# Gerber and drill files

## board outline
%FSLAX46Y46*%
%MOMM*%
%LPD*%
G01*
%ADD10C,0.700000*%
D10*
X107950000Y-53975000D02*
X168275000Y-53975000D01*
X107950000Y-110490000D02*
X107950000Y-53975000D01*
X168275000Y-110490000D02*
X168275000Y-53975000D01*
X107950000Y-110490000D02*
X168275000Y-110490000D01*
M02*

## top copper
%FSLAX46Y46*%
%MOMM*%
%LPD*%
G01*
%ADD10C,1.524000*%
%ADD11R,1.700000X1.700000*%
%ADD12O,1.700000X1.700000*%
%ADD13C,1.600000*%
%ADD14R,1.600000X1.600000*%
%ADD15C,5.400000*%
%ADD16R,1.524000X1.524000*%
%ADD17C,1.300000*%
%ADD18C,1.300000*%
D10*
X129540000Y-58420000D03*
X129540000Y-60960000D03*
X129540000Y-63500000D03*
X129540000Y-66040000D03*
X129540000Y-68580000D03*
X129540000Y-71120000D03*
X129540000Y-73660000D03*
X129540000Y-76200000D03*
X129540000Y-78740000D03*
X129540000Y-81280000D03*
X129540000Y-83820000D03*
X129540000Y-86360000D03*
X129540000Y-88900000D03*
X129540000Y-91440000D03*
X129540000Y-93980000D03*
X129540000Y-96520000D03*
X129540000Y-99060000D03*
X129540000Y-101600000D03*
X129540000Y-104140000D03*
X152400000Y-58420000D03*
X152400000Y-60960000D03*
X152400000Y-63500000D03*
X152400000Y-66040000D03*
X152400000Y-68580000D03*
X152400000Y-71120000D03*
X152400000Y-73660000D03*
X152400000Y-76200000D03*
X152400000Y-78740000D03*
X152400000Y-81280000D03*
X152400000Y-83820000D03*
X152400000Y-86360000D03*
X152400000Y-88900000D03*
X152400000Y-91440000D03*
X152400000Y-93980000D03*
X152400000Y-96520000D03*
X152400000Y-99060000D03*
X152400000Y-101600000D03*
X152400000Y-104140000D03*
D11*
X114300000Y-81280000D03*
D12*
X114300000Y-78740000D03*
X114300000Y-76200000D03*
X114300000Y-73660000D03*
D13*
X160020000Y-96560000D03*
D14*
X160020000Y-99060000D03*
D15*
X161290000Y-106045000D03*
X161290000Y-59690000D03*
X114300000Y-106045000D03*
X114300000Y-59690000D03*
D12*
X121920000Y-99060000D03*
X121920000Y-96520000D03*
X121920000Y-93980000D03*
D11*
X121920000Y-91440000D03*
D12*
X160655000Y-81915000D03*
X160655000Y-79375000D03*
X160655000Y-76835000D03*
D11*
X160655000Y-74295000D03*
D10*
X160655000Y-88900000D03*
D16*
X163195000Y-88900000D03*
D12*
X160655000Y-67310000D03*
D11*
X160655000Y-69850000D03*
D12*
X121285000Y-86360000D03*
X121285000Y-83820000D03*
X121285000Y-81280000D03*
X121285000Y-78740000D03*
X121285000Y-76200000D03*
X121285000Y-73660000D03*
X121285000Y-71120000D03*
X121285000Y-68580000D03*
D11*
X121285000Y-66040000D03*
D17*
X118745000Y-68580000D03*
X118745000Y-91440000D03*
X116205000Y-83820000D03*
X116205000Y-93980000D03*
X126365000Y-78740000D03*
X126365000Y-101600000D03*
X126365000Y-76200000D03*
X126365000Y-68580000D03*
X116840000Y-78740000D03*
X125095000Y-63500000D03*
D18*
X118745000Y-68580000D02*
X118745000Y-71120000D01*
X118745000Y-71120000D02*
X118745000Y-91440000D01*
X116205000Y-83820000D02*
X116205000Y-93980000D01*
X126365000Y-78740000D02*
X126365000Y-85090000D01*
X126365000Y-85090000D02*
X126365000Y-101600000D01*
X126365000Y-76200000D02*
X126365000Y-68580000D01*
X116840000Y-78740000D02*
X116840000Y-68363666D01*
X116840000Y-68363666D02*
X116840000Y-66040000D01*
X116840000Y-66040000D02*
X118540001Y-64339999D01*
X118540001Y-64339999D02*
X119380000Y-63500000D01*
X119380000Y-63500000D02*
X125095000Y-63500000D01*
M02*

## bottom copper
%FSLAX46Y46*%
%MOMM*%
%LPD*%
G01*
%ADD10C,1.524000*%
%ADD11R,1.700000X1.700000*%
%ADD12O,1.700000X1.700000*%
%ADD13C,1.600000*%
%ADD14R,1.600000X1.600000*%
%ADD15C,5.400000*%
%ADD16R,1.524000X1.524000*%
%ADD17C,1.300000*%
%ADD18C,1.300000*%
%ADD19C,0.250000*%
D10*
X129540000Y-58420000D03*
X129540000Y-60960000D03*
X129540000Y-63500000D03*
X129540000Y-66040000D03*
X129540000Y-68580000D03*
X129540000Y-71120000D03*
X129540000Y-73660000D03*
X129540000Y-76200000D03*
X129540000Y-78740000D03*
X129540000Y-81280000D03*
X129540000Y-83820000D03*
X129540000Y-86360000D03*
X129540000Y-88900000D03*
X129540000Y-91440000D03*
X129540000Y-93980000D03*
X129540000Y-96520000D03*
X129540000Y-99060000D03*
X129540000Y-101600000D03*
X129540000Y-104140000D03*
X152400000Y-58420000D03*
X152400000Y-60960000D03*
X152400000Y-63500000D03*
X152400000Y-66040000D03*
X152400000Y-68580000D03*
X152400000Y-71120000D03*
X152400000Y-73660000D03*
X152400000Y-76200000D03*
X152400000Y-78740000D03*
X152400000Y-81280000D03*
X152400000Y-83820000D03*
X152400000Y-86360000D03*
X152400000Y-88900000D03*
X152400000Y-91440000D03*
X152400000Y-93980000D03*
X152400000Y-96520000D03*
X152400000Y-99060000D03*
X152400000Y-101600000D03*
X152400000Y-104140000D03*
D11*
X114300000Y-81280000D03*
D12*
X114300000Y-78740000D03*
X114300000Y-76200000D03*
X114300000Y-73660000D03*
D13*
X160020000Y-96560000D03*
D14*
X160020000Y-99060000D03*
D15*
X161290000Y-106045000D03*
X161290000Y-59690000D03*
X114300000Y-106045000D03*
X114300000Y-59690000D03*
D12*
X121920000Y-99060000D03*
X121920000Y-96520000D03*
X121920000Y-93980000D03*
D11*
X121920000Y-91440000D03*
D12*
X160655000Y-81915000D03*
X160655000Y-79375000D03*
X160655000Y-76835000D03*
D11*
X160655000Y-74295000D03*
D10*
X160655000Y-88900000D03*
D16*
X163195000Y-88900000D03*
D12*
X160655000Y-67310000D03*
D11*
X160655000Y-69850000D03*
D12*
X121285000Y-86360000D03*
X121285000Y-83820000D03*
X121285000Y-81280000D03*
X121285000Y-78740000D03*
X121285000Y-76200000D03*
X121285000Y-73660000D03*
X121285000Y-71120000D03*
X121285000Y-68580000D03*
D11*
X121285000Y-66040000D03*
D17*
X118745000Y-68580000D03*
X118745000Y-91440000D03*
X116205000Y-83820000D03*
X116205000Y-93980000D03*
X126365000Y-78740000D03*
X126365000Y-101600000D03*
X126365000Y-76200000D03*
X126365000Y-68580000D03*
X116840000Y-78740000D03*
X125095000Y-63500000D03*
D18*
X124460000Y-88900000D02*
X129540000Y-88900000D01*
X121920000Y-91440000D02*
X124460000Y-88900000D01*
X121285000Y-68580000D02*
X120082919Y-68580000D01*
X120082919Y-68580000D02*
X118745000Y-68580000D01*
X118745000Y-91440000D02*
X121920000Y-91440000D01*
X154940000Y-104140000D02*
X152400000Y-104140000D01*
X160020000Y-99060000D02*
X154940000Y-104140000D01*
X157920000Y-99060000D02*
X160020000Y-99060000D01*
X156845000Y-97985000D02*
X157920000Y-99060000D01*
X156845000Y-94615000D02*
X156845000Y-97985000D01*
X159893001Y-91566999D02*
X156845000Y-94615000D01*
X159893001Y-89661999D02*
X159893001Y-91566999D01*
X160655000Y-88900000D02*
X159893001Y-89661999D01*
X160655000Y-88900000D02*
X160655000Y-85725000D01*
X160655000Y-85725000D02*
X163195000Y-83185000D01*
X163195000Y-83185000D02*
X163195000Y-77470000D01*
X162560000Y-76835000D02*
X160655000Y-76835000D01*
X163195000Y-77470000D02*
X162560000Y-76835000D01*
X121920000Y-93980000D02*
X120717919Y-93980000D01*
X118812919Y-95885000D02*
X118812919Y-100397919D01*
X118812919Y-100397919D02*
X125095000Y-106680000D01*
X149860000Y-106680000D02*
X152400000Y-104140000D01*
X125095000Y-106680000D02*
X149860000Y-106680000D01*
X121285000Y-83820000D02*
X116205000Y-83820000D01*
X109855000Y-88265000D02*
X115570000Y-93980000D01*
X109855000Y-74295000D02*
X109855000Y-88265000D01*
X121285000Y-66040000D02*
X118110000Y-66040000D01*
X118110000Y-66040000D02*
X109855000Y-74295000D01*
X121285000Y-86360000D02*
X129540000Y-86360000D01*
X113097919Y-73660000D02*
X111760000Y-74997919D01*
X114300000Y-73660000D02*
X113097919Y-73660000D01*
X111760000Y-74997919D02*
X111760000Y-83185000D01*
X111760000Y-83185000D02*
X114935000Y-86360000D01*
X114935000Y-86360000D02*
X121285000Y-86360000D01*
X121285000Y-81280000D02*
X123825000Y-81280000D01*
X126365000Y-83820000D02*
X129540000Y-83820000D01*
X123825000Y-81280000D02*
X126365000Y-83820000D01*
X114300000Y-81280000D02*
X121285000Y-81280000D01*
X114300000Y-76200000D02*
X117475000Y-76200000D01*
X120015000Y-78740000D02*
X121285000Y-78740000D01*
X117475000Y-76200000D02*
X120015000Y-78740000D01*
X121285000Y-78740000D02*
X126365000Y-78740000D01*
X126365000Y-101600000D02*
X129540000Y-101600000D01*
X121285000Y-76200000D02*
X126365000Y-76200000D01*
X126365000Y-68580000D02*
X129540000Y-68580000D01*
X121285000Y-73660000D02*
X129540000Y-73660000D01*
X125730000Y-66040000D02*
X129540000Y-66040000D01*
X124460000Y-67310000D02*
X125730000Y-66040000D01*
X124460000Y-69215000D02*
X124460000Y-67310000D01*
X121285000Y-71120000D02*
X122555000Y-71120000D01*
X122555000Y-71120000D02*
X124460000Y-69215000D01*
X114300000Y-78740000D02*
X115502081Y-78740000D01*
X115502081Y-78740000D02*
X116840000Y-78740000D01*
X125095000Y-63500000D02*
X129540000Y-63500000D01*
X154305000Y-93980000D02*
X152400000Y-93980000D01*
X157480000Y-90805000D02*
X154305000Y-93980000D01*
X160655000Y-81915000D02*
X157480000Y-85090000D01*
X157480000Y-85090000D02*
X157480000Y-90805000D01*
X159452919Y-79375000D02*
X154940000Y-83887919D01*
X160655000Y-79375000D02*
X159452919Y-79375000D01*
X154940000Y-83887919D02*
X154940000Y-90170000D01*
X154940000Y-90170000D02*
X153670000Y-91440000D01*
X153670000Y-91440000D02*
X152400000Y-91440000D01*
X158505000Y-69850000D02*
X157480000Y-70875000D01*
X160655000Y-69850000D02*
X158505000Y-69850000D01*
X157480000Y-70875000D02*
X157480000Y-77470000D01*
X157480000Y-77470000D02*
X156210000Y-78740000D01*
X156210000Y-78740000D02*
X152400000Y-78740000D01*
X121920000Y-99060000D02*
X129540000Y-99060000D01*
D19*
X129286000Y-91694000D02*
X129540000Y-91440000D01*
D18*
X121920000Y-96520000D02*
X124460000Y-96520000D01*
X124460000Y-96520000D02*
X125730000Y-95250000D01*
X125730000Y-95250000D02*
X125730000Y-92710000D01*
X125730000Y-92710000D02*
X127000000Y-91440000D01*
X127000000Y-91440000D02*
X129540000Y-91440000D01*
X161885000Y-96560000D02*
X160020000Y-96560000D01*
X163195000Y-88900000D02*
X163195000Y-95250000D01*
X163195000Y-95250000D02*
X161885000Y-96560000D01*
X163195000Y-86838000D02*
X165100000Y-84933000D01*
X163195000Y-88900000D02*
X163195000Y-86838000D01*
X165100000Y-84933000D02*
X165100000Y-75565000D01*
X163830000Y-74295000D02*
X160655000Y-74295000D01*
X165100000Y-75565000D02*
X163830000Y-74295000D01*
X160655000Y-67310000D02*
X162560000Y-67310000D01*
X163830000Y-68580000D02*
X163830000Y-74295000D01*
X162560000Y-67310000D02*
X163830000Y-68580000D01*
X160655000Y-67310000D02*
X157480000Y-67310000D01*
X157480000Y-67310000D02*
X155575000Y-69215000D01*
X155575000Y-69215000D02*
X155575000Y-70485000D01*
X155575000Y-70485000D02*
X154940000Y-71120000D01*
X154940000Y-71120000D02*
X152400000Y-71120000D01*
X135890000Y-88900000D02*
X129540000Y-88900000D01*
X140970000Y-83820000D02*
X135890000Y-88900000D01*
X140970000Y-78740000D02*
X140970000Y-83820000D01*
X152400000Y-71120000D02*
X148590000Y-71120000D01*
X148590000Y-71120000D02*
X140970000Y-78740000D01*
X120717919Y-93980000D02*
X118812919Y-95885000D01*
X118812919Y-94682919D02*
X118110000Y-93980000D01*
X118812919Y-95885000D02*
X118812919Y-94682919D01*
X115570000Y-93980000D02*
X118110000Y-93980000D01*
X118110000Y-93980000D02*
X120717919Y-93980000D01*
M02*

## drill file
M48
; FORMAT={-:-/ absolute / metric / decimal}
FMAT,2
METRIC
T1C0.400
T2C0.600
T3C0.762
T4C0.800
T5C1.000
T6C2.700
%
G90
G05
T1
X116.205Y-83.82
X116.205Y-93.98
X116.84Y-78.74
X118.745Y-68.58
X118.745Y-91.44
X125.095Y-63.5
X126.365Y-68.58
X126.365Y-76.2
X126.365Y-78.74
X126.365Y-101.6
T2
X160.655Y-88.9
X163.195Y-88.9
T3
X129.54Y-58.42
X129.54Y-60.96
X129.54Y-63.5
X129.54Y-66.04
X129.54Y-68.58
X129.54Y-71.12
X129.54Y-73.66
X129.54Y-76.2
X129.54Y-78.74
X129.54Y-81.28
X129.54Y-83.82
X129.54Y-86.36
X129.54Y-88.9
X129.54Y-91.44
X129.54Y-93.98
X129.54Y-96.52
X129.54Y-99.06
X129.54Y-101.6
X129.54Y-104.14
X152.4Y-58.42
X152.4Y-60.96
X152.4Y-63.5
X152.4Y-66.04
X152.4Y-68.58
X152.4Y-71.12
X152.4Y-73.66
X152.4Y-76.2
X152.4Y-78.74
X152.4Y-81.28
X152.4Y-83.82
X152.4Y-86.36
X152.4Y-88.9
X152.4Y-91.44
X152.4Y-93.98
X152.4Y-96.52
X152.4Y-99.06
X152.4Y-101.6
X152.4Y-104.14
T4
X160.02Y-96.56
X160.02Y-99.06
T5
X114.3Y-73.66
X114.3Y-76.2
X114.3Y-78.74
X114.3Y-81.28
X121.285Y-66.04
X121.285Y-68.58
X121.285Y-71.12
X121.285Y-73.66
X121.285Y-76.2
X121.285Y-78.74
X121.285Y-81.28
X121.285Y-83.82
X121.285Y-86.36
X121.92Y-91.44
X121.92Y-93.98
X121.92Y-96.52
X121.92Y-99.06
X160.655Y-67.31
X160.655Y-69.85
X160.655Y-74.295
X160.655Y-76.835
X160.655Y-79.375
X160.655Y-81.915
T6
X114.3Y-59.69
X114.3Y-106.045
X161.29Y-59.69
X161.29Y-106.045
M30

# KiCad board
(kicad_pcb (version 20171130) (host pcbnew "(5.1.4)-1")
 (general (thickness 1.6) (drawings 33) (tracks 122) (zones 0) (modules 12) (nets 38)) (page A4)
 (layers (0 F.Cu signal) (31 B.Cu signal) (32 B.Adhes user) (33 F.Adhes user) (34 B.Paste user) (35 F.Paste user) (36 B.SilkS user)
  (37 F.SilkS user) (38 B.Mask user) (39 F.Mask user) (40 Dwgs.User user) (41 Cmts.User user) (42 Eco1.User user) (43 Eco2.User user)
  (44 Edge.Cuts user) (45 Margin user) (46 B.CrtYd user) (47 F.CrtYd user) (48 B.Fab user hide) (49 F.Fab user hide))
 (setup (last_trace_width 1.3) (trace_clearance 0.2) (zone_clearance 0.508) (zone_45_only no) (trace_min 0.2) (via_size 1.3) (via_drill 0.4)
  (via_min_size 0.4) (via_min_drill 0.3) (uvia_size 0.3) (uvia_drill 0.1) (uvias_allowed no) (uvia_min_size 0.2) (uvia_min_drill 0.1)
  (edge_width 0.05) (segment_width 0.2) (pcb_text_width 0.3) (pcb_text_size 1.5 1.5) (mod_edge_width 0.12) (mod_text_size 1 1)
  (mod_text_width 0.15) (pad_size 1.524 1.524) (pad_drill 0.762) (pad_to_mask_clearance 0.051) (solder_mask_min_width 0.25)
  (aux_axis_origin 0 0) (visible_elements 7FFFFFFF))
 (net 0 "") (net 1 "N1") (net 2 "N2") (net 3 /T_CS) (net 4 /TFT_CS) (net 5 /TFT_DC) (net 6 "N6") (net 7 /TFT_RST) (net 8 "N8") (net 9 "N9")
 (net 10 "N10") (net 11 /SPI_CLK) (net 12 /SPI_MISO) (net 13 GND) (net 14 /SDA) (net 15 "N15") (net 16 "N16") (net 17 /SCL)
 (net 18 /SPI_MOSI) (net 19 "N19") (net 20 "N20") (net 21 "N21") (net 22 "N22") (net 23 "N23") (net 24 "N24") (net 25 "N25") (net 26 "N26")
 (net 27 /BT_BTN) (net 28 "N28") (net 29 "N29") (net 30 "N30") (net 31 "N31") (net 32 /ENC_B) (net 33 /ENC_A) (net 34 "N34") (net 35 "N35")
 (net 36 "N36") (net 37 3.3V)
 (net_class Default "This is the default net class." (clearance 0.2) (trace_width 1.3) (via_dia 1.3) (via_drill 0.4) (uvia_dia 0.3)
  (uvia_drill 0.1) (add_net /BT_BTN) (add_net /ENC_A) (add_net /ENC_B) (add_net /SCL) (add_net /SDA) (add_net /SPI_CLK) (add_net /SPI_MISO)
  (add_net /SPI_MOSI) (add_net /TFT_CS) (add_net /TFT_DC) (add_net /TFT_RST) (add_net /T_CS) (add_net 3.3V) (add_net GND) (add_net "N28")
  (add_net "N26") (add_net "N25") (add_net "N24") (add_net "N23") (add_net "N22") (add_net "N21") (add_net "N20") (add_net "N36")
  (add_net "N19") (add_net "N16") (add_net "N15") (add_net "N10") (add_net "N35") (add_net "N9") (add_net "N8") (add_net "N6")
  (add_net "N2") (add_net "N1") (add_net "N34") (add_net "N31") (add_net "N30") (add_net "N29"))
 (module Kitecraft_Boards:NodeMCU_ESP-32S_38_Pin (layer F.Cu) (at 140.97 81.28 180)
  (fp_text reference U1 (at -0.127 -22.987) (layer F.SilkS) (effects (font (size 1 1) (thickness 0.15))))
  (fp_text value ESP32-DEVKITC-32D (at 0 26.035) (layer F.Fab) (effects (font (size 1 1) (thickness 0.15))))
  (pad 38 thru_hole circle (at 11.43 22.86 180) (size 1.524 1.524) (drill 0.762) (layers *.Cu *.Mask) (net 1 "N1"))
  (pad 37 thru_hole circle (at 11.43 20.32 180) (size 1.524 1.524) (drill 0.762) (layers *.Cu *.Mask) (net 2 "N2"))
  (pad 36 thru_hole circle (at 11.43 17.78 180) (size 1.524 1.524) (drill 0.762) (layers *.Cu *.Mask) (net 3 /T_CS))
  (pad 35 thru_hole circle (at 11.43 15.24 180) (size 1.524 1.524) (drill 0.762) (layers *.Cu *.Mask) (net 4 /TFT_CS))
  (pad 34 thru_hole circle (at 11.43 12.7 180) (size 1.524 1.524) (drill 0.762) (layers *.Cu *.Mask) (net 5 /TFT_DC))
  (pad 33 thru_hole circle (at 11.43 10.16 180) (size 1.524 1.524) (drill 0.762) (layers *.Cu *.Mask) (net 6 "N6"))
  (pad 32 thru_hole circle (at 11.43 7.62 180) (size 1.524 1.524) (drill 0.762) (layers *.Cu *.Mask) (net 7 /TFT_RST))
  (pad 31 thru_hole circle (at 11.43 5.08 180) (size 1.524 1.524) (drill 0.762) (layers *.Cu *.Mask) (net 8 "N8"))
  (pad 30 thru_hole circle (at 11.43 2.54 180) (size 1.524 1.524) (drill 0.762) (layers *.Cu *.Mask) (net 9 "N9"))
  (pad 29 thru_hole circle (at 11.43 0 180) (size 1.524 1.524) (drill 0.762) (layers *.Cu *.Mask) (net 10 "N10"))
  (pad 28 thru_hole circle (at 11.43 -2.54 180) (size 1.524 1.524) (drill 0.762) (layers *.Cu *.Mask) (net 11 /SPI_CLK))
  (pad 27 thru_hole circle (at 11.43 -5.08 180) (size 1.524 1.524) (drill 0.762) (layers *.Cu *.Mask) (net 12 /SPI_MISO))
  (pad 26 thru_hole circle (at 11.43 -7.62 180) (size 1.524 1.524) (drill 0.762) (layers *.Cu *.Mask) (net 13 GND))
  (pad 25 thru_hole circle (at 11.43 -10.16 180) (size 1.524 1.524) (drill 0.762) (layers *.Cu *.Mask) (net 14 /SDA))
  (pad 24 thru_hole circle (at 11.43 -12.7 180) (size 1.524 1.524) (drill 0.762) (layers *.Cu *.Mask) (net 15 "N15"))
  (pad 23 thru_hole circle (at 11.43 -15.24 180) (size 1.524 1.524) (drill 0.762) (layers *.Cu *.Mask) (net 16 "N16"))
  (pad 22 thru_hole circle (at 11.43 -17.78 180) (size 1.524 1.524) (drill 0.762) (layers *.Cu *.Mask) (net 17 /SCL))
  (pad 21 thru_hole circle (at 11.43 -20.32 180) (size 1.524 1.524) (drill 0.762) (layers *.Cu *.Mask) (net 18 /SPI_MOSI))
  (pad 20 thru_hole circle (at 11.43 -22.86 180) (size 1.524 1.524) (drill 0.762) (layers *.Cu *.Mask) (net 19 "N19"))
  (pad 19 thru_hole circle (at -11.43 22.86 180) (size 1.524 1.524) (drill 0.762) (layers *.Cu *.Mask) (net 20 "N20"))
  (pad 18 thru_hole circle (at -11.43 20.32 180) (size 1.524 1.524) (drill 0.762) (layers *.Cu *.Mask) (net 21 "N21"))
  (pad 17 thru_hole circle (at -11.43 17.78 180) (size 1.524 1.524) (drill 0.762) (layers *.Cu *.Mask) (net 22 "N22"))
  (pad 16 thru_hole circle (at -11.43 15.24 180) (size 1.524 1.524) (drill 0.762) (layers *.Cu *.Mask) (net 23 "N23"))
  (pad 15 thru_hole circle (at -11.43 12.7 180) (size 1.524 1.524) (drill 0.762) (layers *.Cu *.Mask) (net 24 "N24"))
  (pad 14 thru_hole circle (at -11.43 10.16 180) (size 1.524 1.524) (drill 0.762) (layers *.Cu *.Mask) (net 13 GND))
  (pad 13 thru_hole circle (at -11.43 7.62 180) (size 1.524 1.524) (drill 0.762) (layers *.Cu *.Mask) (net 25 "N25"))
  (pad 12 thru_hole circle (at -11.43 5.08 180) (size 1.524 1.524) (drill 0.762) (layers *.Cu *.Mask) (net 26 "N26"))
  (pad 11 thru_hole circle (at -11.43 2.54 180) (size 1.524 1.524) (drill 0.762) (layers *.Cu *.Mask) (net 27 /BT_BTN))
  (pad 10 thru_hole circle (at -11.43 0 180) (size 1.524 1.524) (drill 0.762) (layers *.Cu *.Mask) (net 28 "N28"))
  (pad 9 thru_hole circle (at -11.43 -2.54 180) (size 1.524 1.524) (drill 0.762) (layers *.Cu *.Mask) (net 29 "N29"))
  (pad 8 thru_hole circle (at -11.43 -5.08 180) (size 1.524 1.524) (drill 0.762) (layers *.Cu *.Mask) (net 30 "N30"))
  (pad 7 thru_hole circle (at -11.43 -7.62 180) (size 1.524 1.524) (drill 0.762) (layers *.Cu *.Mask) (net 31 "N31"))
  (pad 6 thru_hole circle (at -11.43 -10.16 180) (size 1.524 1.524) (drill 0.762) (layers *.Cu *.Mask) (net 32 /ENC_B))
  (pad 5 thru_hole circle (at -11.43 -12.7 180) (size 1.524 1.524) (drill 0.762) (layers *.Cu *.Mask) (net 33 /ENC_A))
  (pad 4 thru_hole circle (at -11.43 -15.24 180) (size 1.524 1.524) (drill 0.762) (layers *.Cu *.Mask) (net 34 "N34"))
  (pad 3 thru_hole circle (at -11.43 -17.78 180) (size 1.524 1.524) (drill 0.762) (layers *.Cu *.Mask) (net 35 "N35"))
  (pad 2 thru_hole circle (at -11.43 -20.32 180) (size 1.524 1.524) (drill 0.762) (layers *.Cu *.Mask) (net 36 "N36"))
  (pad 1 thru_hole circle (at -11.43 -22.86 180) (size 1.524 1.524) (drill 0.762) (layers *.Cu *.Mask) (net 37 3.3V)))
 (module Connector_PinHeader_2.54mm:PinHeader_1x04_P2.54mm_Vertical (layer F.Cu) (at 114.3 81.28 180)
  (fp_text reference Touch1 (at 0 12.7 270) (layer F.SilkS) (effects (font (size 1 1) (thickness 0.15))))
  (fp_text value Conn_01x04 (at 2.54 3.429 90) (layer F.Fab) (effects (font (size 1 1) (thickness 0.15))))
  (pad 1 thru_hole rect (at 0 0 180) (size 1.7 1.7) (drill 1) (layers *.Cu *.Mask) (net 11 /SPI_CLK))
  (pad 2 thru_hole oval (at 0 2.54 180) (size 1.7 1.7) (drill 1) (layers *.Cu *.Mask) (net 3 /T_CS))
  (pad 3 thru_hole oval (at 0 5.08 180) (size 1.7 1.7) (drill 1) (layers *.Cu *.Mask) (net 18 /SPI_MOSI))
  (pad 4 thru_hole oval (at 0 7.62 180) (size 1.7 1.7) (drill 1) (layers *.Cu *.Mask) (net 12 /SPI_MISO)))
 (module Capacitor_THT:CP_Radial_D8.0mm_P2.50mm (layer F.Cu) (at 160.02 99.06 90)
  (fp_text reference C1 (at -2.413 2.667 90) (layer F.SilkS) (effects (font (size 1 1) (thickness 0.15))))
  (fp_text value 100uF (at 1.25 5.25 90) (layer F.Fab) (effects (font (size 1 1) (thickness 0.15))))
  (pad 2 thru_hole circle (at 2.5 0 90) (size 1.6 1.6) (drill 0.8) (layers *.Cu *.Mask) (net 13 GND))
  (pad 1 thru_hole rect (at 0 0 90) (size 1.6 1.6) (drill 0.8) (layers *.Cu *.Mask) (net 37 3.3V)))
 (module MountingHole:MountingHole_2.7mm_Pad (layer F.Cu) (at 161.29 106.045)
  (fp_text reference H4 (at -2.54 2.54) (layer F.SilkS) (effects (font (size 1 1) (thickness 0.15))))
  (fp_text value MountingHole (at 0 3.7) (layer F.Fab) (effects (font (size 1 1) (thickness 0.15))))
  (pad 1 thru_hole circle (at 0 0) (size 5.4 5.4) (drill 2.7) (layers *.Cu *.Mask)))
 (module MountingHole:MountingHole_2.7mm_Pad (layer F.Cu) (at 161.29 59.69)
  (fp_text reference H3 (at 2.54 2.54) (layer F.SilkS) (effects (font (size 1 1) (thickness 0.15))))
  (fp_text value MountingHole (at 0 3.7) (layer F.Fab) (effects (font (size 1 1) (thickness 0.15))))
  (pad 1 thru_hole circle (at 0 0) (size 5.4 5.4) (drill 2.7) (layers *.Cu *.Mask)))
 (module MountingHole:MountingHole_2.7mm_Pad (layer F.Cu) (at 114.3 106.045)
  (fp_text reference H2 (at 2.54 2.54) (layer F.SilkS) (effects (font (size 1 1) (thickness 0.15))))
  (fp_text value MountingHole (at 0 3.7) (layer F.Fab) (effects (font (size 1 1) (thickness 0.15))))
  (pad 1 thru_hole circle (at 0 0) (size 5.4 5.4) (drill 2.7) (layers *.Cu *.Mask)))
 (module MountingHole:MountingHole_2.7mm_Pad (layer F.Cu) (at 114.3 59.69)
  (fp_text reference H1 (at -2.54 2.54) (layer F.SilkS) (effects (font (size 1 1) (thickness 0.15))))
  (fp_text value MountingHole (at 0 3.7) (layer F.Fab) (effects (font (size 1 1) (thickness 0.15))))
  (pad 1 thru_hole circle (at 0 0) (size 5.4 5.4) (drill 2.7) (layers *.Cu *.Mask)))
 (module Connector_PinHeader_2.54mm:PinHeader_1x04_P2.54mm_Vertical (layer F.Cu) (at 121.92 91.44)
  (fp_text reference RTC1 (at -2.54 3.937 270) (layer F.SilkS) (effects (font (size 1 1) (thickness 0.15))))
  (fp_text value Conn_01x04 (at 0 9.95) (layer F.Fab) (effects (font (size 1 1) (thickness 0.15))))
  (pad 4 thru_hole oval (at 0 7.62) (size 1.7 1.7) (drill 1) (layers *.Cu *.Mask) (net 17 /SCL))
  (pad 3 thru_hole oval (at 0 5.08) (size 1.7 1.7) (drill 1) (layers *.Cu *.Mask) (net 14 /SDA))
  (pad 2 thru_hole oval (at 0 2.54) (size 1.7 1.7) (drill 1) (layers *.Cu *.Mask) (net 37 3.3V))
  (pad 1 thru_hole rect (at 0 0) (size 1.7 1.7) (drill 1) (layers *.Cu *.Mask) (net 13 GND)))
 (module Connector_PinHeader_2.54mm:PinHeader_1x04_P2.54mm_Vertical (layer F.Cu) (at 160.655 74.295)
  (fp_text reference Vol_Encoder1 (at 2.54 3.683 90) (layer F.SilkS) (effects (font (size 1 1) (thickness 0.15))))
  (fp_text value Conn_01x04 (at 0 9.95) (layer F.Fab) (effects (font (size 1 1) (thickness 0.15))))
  (pad 4 thru_hole oval (at 0 7.62) (size 1.7 1.7) (drill 1) (layers *.Cu *.Mask) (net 33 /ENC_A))
  (pad 3 thru_hole oval (at 0 5.08) (size 1.7 1.7) (drill 1) (layers *.Cu *.Mask) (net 32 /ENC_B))
  (pad 2 thru_hole oval (at 0 2.54) (size 1.7 1.7) (drill 1) (layers *.Cu *.Mask) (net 37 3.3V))
  (pad 1 thru_hole rect (at 0 0) (size 1.7 1.7) (drill 1) (layers *.Cu *.Mask) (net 13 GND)))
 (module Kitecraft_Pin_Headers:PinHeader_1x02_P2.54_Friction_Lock (layer F.Cu) (at 160.655 88.9 270)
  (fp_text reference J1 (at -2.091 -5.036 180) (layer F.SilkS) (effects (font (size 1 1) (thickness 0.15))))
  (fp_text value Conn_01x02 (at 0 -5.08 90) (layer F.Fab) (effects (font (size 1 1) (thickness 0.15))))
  (pad 2 thru_hole circle (at 0 0 270) (size 1.524 1.524) (drill 0.6) (layers *.Cu *.Mask) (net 37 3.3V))
  (pad 1 thru_hole rect (at 0 -2.54 270) (size 1.524 1.524) (drill 0.6) (layers *.Cu *.Mask) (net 13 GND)))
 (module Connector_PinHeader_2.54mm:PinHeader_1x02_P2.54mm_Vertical (layer F.Cu) (at 160.655 69.85 180)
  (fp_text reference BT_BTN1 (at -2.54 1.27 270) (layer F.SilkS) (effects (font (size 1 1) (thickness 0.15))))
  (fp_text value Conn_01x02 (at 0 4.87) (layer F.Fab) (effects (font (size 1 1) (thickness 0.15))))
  (pad 2 thru_hole oval (at 0 2.54 180) (size 1.7 1.7) (drill 1) (layers *.Cu *.Mask) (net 13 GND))
  (pad 1 thru_hole rect (at 0 0 180) (size 1.7 1.7) (drill 1) (layers *.Cu *.Mask) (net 27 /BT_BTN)))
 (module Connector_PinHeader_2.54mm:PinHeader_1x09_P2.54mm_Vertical (layer F.Cu) (at 121.285 66.04)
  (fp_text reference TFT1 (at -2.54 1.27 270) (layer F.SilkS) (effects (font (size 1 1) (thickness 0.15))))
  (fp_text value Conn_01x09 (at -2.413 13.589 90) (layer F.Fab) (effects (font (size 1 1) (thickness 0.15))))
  (pad 9 thru_hole oval (at 0 20.32) (size 1.7 1.7) (drill 1) (layers *.Cu *.Mask) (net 12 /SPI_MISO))
  (pad 8 thru_hole oval (at 0 17.78) (size 1.7 1.7) (drill 1) (layers *.Cu *.Mask) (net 37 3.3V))
  (pad 7 thru_hole oval (at 0 15.24) (size 1.7 1.7) (drill 1) (layers *.Cu *.Mask) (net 11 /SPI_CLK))
  (pad 6 thru_hole oval (at 0 12.7) (size 1.7 1.7) (drill 1) (layers *.Cu *.Mask) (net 18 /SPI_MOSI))
  (pad 5 thru_hole oval (at 0 10.16) (size 1.7 1.7) (drill 1) (layers *.Cu *.Mask) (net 5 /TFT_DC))
  (pad 4 thru_hole oval (at 0 7.62) (size 1.7 1.7) (drill 1) (layers *.Cu *.Mask) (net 7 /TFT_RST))
  (pad 3 thru_hole oval (at 0 5.08) (size 1.7 1.7) (drill 1) (layers *.Cu *.Mask) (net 4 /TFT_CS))
  (pad 2 thru_hole oval (at 0 2.54) (size 1.7 1.7) (drill 1) (layers *.Cu *.Mask) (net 13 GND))
  (pad 1 thru_hole rect (at 0 0) (size 1.7 1.7) (drill 1) (layers *.Cu *.Mask) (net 37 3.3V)))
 (gr_line (start 107.95 53.975) (end 168.275 53.975) (layer Edge.Cuts) (width 0.7))
 (gr_line (start 107.95 110.49) (end 107.95 53.975) (layer Edge.Cuts) (width 0.7))
 (gr_line (start 168.275 110.49) (end 168.275 53.975) (layer Edge.Cuts) (width 0.7))
 (gr_line (start 107.95 110.49) (end 168.275 110.49) (layer Edge.Cuts) (width 0.7))
 (segment (start 124.46 88.9) (end 129.54 88.9) (width 1.3) (layer B.Cu) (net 13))
 (segment (start 121.92 91.44) (end 124.46 88.9) (width 1.3) (layer B.Cu) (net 13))
 (segment (start 121.285 68.58) (end 120.082919 68.58) (width 1.3) (layer B.Cu) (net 13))
 (via (at 118.745 68.58) (size 1.3) (drill 0.4) (layers F.Cu B.Cu) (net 13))
 (segment (start 120.082919 68.58) (end 118.745 68.58) (width 1.3) (layer B.Cu) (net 13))
 (segment (start 118.745 68.58) (end 118.745 71.12) (width 1.3) (layer F.Cu) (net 13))
 (segment (start 118.745 71.12) (end 118.745 91.44) (width 1.3) (layer F.Cu) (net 13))
 (via (at 118.745 91.44) (size 1.3) (drill 0.4) (layers F.Cu B.Cu) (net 13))
 (segment (start 118.745 91.44) (end 121.92 91.44) (width 1.3) (layer B.Cu) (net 13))
 (segment (start 154.94 104.14) (end 152.4 104.14) (width 1.3) (layer B.Cu) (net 37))
 (segment (start 160.02 99.06) (end 154.94 104.14) (width 1.3) (layer B.Cu) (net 37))
 (segment (start 157.92 99.06) (end 160.02 99.06) (width 1.3) (layer B.Cu) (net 37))
 (segment (start 156.845 97.985) (end 157.92 99.06) (width 1.3) (layer B.Cu) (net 37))
 (segment (start 156.845 94.615) (end 156.845 97.985) (width 1.3) (layer B.Cu) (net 37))
 (segment (start 159.893001 91.566999) (end 156.845 94.615) (width 1.3) (layer B.Cu) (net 37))
 (segment (start 159.893001 89.661999) (end 159.893001 91.566999) (width 1.3) (layer B.Cu) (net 37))
 (segment (start 160.655 88.9) (end 159.893001 89.661999) (width 1.3) (layer B.Cu) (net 37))
 (segment (start 160.655 88.9) (end 160.655 85.725) (width 1.3) (layer B.Cu) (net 37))
 (segment (start 160.655 85.725) (end 163.195 83.185) (width 1.3) (layer B.Cu) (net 37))
 (segment (start 163.195 83.185) (end 163.195 77.47) (width 1.3) (layer B.Cu) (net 37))
 (segment (start 162.56 76.835) (end 160.655 76.835) (width 1.3) (layer B.Cu) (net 37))
 (segment (start 163.195 77.47) (end 162.56 76.835) (width 1.3) (layer B.Cu) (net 37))
 (segment (start 121.92 93.98) (end 120.717919 93.98) (width 1.3) (layer B.Cu) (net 37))
 (segment (start 118.812919 95.885) (end 118.812919 100.397919) (width 1.3) (layer B.Cu) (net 37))
 (segment (start 118.812919 100.397919) (end 125.095 106.68) (width 1.3) (layer B.Cu) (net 37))
 (segment (start 149.86 106.68) (end 152.4 104.14) (width 1.3) (layer B.Cu) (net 37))
 (segment (start 125.095 106.68) (end 149.86 106.68) (width 1.3) (layer B.Cu) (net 37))
 (segment (start 121.285 83.82) (end 116.205 83.82) (width 1.3) (layer B.Cu) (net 37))
 (via (at 116.205 83.82) (size 1.3) (drill 0.4) (layers F.Cu B.Cu) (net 37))
 (segment (start 116.205 83.82) (end 116.205 93.98) (width 1.3) (layer F.Cu) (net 37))
 (via (at 116.205 93.98) (size 1.3) (drill 0.4) (layers F.Cu B.Cu) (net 37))
 (segment (start 109.855 88.265) (end 115.57 93.98) (width 1.3) (layer B.Cu) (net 37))
 (segment (start 109.855 74.295) (end 109.855 88.265) (width 1.3) (layer B.Cu) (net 37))
 (segment (start 121.285 66.04) (end 118.11 66.04) (width 1.3) (layer B.Cu) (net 37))
 (segment (start 118.11 66.04) (end 109.855 74.295) (width 1.3) (layer B.Cu) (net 37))
 (segment (start 121.285 86.36) (end 129.54 86.36) (width 1.3) (layer B.Cu) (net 12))
 (segment (start 113.097919 73.66) (end 111.76 74.997919) (width 1.3) (layer B.Cu) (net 12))
 (segment (start 114.3 73.66) (end 113.097919 73.66) (width 1.3) (layer B.Cu) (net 12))
 (segment (start 111.76 74.997919) (end 111.76 83.185) (width 1.3) (layer B.Cu) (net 12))
 (segment (start 111.76 83.185) (end 114.935 86.36) (width 1.3) (layer B.Cu) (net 12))
 (segment (start 114.935 86.36) (end 121.285 86.36) (width 1.3) (layer B.Cu) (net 12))
 (segment (start 121.285 81.28) (end 123.825 81.28) (width 1.3) (layer B.Cu) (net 11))
 (segment (start 126.365 83.82) (end 129.54 83.82) (width 1.3) (layer B.Cu) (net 11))
 (segment (start 123.825 81.28) (end 126.365 83.82) (width 1.3) (layer B.Cu) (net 11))
 (segment (start 114.3 81.28) (end 121.285 81.28) (width 1.3) (layer B.Cu) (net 11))
 (segment (start 114.3 76.2) (end 117.475 76.2) (width 1.3) (layer B.Cu) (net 18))
 (segment (start 120.015 78.74) (end 121.285 78.74) (width 1.3) (layer B.Cu) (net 18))
 (segment (start 117.475 76.2) (end 120.015 78.74) (width 1.3) (layer B.Cu) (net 18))
 (segment (start 121.285 78.74) (end 126.365 78.74) (width 1.3) (layer B.Cu) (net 18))
 (via (at 126.365 78.74) (size 1.3) (drill 0.4) (layers F.Cu B.Cu) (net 18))
 (segment (start 126.365 78.74) (end 126.365 85.09) (width 1.3) (layer F.Cu) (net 18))
 (segment (start 126.365 85.09) (end 126.365 101.6) (width 1.3) (layer F.Cu) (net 18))
 (via (at 126.365 101.6) (size 1.3) (drill 0.4) (layers F.Cu B.Cu) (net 18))
 (segment (start 126.365 101.6) (end 129.54 101.6) (width 1.3) (layer B.Cu) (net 18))
 (segment (start 121.285 76.2) (end 126.365 76.2) (width 1.3) (layer B.Cu) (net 5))
 (via (at 126.365 76.2) (size 1.3) (drill 0.4) (layers F.Cu B.Cu) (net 5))
 (segment (start 126.365 76.2) (end 126.365 68.58) (width 1.3) (layer F.Cu) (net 5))
 (via (at 126.365 68.58) (size 1.3) (drill 0.4) (layers F.Cu B.Cu) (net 5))
 (segment (start 126.365 68.58) (end 129.54 68.58) (width 1.3) (layer B.Cu) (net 5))
 (segment (start 121.285 73.66) (end 129.54 73.66) (width 1.3) (layer B.Cu) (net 7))
 (segment (start 125.73 66.04) (end 129.54 66.04) (width 1.3) (layer B.Cu) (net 4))
 (segment (start 124.46 67.31) (end 125.73 66.04) (width 1.3) (layer B.Cu) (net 4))
 (segment (start 124.46 69.215) (end 124.46 67.31) (width 1.3) (layer B.Cu) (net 4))
 (segment (start 121.285 71.12) (end 122.555 71.12) (width 1.3) (layer B.Cu) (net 4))
 (segment (start 122.555 71.12) (end 124.46 69.215) (width 1.3) (layer B.Cu) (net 4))
 (segment (start 114.3 78.74) (end 115.502081 78.74) (width 1.3) (layer B.Cu) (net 3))
 (via (at 116.84 78.74) (size 1.3) (drill 0.4) (layers F.Cu B.Cu) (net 3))
 (segment (start 115.502081 78.74) (end 116.84 78.74) (width 1.3) (layer B.Cu) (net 3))
 (segment (start 116.84 78.74) (end 116.84 68.363666) (width 1.3) (layer F.Cu) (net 3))
 (segment (start 116.84 68.363666) (end 116.84 66.04) (width 1.3) (layer F.Cu) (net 3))
 (segment (start 116.84 66.04) (end 118.540001 64.339999) (width 1.3) (layer F.Cu) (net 3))
 (segment (start 118.540001 64.339999) (end 119.38 63.5) (width 1.3) (layer F.Cu) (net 3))
 (via (at 125.095 63.5) (size 1.3) (drill 0.4) (layers F.Cu B.Cu) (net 3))
 (segment (start 119.38 63.5) (end 125.095 63.5) (width 1.3) (layer F.Cu) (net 3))
 (segment (start 125.095 63.5) (end 129.54 63.5) (width 1.3) (layer B.Cu) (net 3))
 (segment (start 154.305 93.98) (end 152.4 93.98) (width 1.3) (layer B.Cu) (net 33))
 (segment (start 157.48 90.805) (end 154.305 93.98) (width 1.3) (layer B.Cu) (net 33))
 (segment (start 160.655 81.915) (end 157.48 85.09) (width 1.3) (layer B.Cu) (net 33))
 (segment (start 157.48 85.09) (end 157.48 90.805) (width 1.3) (layer B.Cu) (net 33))
 (segment (start 159.452919 79.375) (end 154.94 83.887919) (width 1.3) (layer B.Cu) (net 32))
 (segment (start 160.655 79.375) (end 159.452919 79.375) (width 1.3) (layer B.Cu) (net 32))
 (segment (start 154.94 83.887919) (end 154.94 90.17) (width 1.3) (layer B.Cu) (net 32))
 (segment (start 154.94 90.17) (end 153.67 91.44) (width 1.3) (layer B.Cu) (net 32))
 (segment (start 153.67 91.44) (end 152.4 91.44) (width 1.3) (layer B.Cu) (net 32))
 (segment (start 158.505 69.85) (end 157.48 70.875) (width 1.3) (layer B.Cu) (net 27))
 (segment (start 160.655 69.85) (end 158.505 69.85) (width 1.3) (layer B.Cu) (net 27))
 (segment (start 157.48 70.875) (end 157.48 77.47) (width 1.3) (layer B.Cu) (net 27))
 (segment (start 157.48 77.47) (end 156.21 78.74) (width 1.3) (layer B.Cu) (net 27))
 (segment (start 156.21 78.74) (end 152.4 78.74) (width 1.3) (layer B.Cu) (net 27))
 (segment (start 121.92 99.06) (end 129.54 99.06) (width 1.3) (layer B.Cu) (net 17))
 (segment (start 129.286 91.694) (end 129.54 91.44) (width 0.25) (layer B.Cu) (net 14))
 (segment (start 121.92 96.52) (end 124.46 96.52) (width 1.3) (layer B.Cu) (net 14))
 (segment (start 124.46 96.52) (end 125.73 95.25) (width 1.3) (layer B.Cu) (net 14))
 (segment (start 125.73 95.25) (end 125.73 92.71) (width 1.3) (layer B.Cu) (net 14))
 (segment (start 125.73 92.71) (end 127 91.44) (width 1.3) (layer B.Cu) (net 14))
 (segment (start 127 91.44) (end 129.54 91.44) (width 1.3) (layer B.Cu) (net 14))
 (segment (start 161.885 96.56) (end 160.02 96.56) (width 1.3) (layer B.Cu) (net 13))
 (segment (start 163.195 88.9) (end 163.195 95.25) (width 1.3) (layer B.Cu) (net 13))
 (segment (start 163.195 95.25) (end 161.885 96.56) (width 1.3) (layer B.Cu) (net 13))
 (segment (start 163.195 86.838) (end 165.1 84.933) (width 1.3) (layer B.Cu) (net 13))
 (segment (start 163.195 88.9) (end 163.195 86.838) (width 1.3) (layer B.Cu) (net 13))
 (segment (start 165.1 84.933) (end 165.1 75.565) (width 1.3) (layer B.Cu) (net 13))
 (segment (start 163.83 74.295) (end 160.655 74.295) (width 1.3) (layer B.Cu) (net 13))
 (segment (start 165.1 75.565) (end 163.83 74.295) (width 1.3) (layer B.Cu) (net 13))
 (segment (start 160.655 67.31) (end 162.56 67.31) (width 1.3) (layer B.Cu) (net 13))
 (segment (start 163.83 68.58) (end 163.83 74.295) (width 1.3) (layer B.Cu) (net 13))
 (segment (start 162.56 67.31) (end 163.83 68.58) (width 1.3) (layer B.Cu) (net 13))
 (segment (start 160.655 67.31) (end 157.48 67.31) (width 1.3) (layer B.Cu) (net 13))
 (segment (start 157.48 67.31) (end 155.575 69.215) (width 1.3) (layer B.Cu) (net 13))
 (segment (start 155.575 69.215) (end 155.575 70.485) (width 1.3) (layer B.Cu) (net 13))
 (segment (start 155.575 70.485) (end 154.94 71.12) (width 1.3) (layer B.Cu) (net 13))
 (segment (start 154.94 71.12) (end 152.4 71.12) (width 1.3) (layer B.Cu) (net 13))
 (segment (start 135.89 88.9) (end 129.54 88.9) (width 1.3) (layer B.Cu) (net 13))
 (segment (start 140.97 83.82) (end 135.89 88.9) (width 1.3) (layer B.Cu) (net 13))
 (segment (start 140.97 78.74) (end 140.97 83.82) (width 1.3) (layer B.Cu) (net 13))
 (segment (start 152.4 71.12) (end 148.59 71.12) (width 1.3) (layer B.Cu) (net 13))
 (segment (start 148.59 71.12) (end 140.97 78.74) (width 1.3) (layer B.Cu) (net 13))
 (segment (start 120.717919 93.98) (end 118.812919 95.885) (width 1.3) (layer B.Cu) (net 37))
 (segment (start 118.812919 94.682919) (end 118.11 93.98) (width 1.3) (layer B.Cu) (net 37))
 (segment (start 118.812919 95.885) (end 118.812919 94.682919) (width 1.3) (layer B.Cu) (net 37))
 (segment (start 115.57 93.98) (end 118.11 93.98) (width 1.3) (layer B.Cu) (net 37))
 (segment (start 118.11 93.98) (end 120.717919 93.98) (width 1.3) (layer B.Cu) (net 37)))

